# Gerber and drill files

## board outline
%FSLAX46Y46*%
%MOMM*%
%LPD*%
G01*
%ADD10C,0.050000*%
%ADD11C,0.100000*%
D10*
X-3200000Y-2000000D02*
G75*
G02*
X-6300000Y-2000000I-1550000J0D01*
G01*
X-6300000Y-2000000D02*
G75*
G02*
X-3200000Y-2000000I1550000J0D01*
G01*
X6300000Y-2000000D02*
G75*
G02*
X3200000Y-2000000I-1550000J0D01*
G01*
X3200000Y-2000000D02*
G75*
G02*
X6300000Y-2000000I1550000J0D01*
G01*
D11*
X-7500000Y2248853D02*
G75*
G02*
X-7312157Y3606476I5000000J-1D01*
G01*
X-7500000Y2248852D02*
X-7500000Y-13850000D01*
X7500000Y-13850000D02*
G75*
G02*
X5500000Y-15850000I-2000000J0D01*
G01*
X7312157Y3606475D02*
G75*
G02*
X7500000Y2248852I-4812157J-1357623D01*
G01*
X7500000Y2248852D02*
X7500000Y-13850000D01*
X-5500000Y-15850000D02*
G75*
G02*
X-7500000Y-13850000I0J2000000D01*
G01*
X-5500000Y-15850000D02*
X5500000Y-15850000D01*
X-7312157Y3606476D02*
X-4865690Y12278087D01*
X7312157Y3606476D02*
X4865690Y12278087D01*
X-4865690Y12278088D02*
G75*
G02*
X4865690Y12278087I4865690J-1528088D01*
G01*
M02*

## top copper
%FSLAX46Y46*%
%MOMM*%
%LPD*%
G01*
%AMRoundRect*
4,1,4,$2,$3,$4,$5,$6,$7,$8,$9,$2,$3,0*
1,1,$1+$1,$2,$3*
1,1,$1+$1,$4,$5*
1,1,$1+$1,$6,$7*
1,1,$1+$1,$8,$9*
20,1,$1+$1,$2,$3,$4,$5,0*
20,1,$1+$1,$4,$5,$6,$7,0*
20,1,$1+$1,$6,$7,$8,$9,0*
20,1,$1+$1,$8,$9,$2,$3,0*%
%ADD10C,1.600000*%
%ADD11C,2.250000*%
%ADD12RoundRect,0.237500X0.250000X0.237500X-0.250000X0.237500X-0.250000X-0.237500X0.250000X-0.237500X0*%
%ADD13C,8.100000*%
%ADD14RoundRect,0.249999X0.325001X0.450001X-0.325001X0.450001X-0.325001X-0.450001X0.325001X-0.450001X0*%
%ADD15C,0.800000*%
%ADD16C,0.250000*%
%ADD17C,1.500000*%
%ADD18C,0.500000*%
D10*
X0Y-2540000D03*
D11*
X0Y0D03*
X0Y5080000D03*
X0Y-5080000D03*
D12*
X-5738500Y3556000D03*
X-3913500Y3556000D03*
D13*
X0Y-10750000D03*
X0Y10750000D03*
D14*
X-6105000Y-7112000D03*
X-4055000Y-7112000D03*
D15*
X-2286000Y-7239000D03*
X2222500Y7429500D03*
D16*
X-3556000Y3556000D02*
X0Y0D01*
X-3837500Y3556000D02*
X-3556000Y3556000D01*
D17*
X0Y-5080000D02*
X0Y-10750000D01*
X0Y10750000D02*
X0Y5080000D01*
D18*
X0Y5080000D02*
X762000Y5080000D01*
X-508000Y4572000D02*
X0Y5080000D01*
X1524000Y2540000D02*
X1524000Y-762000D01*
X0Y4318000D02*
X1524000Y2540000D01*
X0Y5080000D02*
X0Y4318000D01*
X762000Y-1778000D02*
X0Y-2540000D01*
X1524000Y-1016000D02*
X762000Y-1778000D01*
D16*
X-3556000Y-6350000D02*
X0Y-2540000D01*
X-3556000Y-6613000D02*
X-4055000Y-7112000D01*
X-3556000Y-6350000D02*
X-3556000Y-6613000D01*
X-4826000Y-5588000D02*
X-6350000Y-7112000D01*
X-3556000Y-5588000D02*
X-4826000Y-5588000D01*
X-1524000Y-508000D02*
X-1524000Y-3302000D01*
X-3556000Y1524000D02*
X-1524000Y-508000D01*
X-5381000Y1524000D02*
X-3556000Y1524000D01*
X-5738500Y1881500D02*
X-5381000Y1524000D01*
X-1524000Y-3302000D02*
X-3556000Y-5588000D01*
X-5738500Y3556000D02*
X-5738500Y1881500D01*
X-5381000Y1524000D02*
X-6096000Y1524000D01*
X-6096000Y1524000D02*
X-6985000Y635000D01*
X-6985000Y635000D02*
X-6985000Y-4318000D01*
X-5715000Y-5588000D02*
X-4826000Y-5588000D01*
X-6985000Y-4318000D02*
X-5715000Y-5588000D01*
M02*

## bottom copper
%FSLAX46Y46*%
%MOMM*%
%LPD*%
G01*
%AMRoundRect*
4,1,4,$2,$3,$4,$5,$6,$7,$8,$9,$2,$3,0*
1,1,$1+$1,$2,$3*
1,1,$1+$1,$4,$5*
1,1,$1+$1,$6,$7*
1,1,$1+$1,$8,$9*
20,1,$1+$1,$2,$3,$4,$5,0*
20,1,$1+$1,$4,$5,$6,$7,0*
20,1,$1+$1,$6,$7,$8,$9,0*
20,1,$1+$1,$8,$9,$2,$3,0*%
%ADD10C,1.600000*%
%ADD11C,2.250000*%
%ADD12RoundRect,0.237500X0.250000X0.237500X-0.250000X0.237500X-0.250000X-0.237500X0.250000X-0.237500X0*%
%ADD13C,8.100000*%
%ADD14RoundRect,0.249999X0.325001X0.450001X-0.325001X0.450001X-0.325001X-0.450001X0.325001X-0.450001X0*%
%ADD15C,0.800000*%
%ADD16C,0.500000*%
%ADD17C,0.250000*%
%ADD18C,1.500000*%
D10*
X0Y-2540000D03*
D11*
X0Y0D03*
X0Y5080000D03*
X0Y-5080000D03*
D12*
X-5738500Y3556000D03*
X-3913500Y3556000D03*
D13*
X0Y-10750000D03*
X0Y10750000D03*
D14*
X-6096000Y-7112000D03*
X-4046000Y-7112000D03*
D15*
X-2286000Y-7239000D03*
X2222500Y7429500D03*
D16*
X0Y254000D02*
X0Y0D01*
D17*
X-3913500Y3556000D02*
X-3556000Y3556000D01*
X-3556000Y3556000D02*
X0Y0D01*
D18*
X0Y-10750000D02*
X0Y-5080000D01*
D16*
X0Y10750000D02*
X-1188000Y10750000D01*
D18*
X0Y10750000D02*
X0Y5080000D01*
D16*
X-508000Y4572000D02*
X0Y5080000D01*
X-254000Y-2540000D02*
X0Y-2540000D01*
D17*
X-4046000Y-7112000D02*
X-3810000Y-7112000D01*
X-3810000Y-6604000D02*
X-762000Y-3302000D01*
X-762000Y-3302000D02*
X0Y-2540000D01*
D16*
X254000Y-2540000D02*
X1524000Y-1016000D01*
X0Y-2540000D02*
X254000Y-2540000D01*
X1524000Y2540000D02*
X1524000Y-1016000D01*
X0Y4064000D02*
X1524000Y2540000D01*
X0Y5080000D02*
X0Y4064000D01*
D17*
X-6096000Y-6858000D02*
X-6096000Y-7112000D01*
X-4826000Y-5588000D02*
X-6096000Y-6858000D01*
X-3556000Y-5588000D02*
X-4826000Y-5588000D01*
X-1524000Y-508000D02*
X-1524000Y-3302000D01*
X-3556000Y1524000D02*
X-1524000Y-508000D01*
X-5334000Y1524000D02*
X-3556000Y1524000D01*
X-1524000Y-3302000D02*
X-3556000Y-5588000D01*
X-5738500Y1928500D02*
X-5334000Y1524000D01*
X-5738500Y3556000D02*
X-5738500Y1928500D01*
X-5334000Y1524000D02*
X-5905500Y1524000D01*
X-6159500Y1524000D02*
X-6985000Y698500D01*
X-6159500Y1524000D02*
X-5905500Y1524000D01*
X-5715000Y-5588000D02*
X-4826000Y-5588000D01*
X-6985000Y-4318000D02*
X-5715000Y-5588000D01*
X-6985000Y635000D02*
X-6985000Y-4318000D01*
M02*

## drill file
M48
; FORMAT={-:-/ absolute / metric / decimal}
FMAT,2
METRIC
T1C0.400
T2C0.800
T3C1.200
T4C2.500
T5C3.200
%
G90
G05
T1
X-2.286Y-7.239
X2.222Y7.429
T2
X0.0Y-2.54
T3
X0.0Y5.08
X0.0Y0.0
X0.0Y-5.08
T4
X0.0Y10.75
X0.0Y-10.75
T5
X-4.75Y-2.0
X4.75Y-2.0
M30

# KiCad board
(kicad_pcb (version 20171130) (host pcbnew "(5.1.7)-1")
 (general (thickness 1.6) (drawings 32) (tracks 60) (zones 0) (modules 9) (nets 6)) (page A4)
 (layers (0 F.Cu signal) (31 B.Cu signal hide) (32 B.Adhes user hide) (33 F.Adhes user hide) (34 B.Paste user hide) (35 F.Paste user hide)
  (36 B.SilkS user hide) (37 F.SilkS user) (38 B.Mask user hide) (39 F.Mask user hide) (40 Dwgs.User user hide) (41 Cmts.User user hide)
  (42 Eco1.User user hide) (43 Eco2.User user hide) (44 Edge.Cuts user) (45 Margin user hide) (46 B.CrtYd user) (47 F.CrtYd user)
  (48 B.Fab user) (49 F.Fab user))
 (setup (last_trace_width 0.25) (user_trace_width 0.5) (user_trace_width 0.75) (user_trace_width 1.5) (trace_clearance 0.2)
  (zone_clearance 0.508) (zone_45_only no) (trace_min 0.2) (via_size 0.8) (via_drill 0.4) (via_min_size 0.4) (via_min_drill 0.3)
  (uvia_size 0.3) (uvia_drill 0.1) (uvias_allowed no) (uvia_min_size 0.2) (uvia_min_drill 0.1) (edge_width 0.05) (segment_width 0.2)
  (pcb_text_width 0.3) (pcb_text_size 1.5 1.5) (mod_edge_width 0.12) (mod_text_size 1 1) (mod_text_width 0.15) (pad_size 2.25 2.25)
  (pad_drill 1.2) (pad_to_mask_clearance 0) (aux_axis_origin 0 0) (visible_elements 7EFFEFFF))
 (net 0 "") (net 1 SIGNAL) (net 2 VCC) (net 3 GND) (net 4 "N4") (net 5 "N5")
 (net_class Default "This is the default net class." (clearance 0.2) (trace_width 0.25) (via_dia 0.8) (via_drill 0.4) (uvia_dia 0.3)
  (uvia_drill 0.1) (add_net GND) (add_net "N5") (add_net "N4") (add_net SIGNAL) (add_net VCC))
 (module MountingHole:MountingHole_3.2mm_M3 (layer F.Cu) (at 4.75 2)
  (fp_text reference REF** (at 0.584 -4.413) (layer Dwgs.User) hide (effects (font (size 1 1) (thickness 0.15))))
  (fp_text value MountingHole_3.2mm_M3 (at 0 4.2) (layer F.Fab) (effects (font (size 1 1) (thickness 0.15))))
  (pad 1 np_thru_hole circle (at 0 0) (size 3.2 3.2) (drill 3.2) (layers *.Cu *.Mask)))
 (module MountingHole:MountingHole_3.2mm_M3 (layer F.Cu) (at -4.75 2)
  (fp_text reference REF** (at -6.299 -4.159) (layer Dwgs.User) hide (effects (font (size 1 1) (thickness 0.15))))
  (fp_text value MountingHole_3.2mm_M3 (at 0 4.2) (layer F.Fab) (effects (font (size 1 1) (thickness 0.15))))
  (pad 1 np_thru_hole circle (at 0 0) (size 3.2 3.2) (drill 3.2) (layers *.Cu *.Mask)))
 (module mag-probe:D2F (layer F.Cu) (at 0 0 270)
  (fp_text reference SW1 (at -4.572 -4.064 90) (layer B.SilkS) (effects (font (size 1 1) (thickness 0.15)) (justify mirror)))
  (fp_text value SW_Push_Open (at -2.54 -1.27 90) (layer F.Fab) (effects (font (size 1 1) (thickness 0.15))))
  (pad 4 thru_hole circle (at 2.54 0 270) (size 1.6 1.6) (drill 0.8) (layers *.Cu *.Mask) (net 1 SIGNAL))
  (pad 3 thru_hole circle (at 0 0 270) (size 2.25 2.25) (drill 1.2) (layers *.Cu *.Mask) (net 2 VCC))
  (pad 2 thru_hole circle (at -5.08 0 270) (size 2.25 2.25) (drill 1.2) (layers *.Cu *.Mask) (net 1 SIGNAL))
  (pad 1 thru_hole circle (at 5.08 0 270) (size 2.25 2.25) (drill 1.2) (layers *.Cu *.Mask) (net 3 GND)))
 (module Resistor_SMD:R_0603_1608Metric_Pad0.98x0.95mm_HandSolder (layer B.Cu) (at -4.826 -3.556 180)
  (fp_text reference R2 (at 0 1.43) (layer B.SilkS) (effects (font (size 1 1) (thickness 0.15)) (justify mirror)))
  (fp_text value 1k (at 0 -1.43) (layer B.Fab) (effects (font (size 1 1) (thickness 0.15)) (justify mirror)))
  (pad 2 smd roundrect (at 0.9125 0 180) (size 0.975 0.95) (layers B.Cu B.Paste B.Mask) (roundrect_rratio 0.25) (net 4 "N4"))
  (pad 1 smd roundrect (at -0.9125 0 180) (size 0.975 0.95) (layers B.Cu B.Paste B.Mask) (roundrect_rratio 0.25) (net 2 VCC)))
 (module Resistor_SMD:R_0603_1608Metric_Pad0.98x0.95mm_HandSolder (layer F.Cu) (at -4.826 -3.556 180)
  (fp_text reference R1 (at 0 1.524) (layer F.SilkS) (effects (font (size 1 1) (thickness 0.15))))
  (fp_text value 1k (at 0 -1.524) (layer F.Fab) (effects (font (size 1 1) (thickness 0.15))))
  (pad 2 smd roundrect (at 0.9125 0 180) (size 0.975 0.95) (layers F.Cu F.Paste F.Mask) (roundrect_rratio 0.25) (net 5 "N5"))
  (pad 1 smd roundrect (at -0.9125 0 180) (size 0.975 0.95) (layers F.Cu F.Paste F.Mask) (roundrect_rratio 0.25) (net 2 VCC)))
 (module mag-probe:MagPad (layer F.Cu) (at 0 10.75)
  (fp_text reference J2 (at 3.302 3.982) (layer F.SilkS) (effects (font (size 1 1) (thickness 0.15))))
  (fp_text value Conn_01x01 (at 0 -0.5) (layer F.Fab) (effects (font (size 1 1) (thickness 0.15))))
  (pad 1 thru_hole circle (at 0 0) (size 8.1 8.1) (drill 2.5) (layers *.Cu *.Mask) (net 3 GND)))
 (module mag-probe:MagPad (layer F.Cu) (at 0 -10.75)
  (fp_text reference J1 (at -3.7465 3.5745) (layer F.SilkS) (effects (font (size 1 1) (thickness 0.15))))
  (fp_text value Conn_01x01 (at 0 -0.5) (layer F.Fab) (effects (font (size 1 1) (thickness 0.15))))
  (pad 1 thru_hole circle (at 0 0) (size 8.1 8.1) (drill 2.5) (layers *.Cu *.Mask) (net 1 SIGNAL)))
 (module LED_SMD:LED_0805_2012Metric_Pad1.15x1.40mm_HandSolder (layer B.Cu) (at -5.071 7.112 180)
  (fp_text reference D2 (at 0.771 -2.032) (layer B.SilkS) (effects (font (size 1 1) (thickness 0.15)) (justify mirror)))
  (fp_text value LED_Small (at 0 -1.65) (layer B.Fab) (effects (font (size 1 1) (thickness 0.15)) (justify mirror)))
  (pad 2 smd roundrect (at 1.025 0 180) (size 1.15 1.4) (layers B.Cu B.Paste B.Mask) (roundrect_rratio 0.2173904347826087) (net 4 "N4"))
  (pad 1 smd roundrect (at -1.025 0 180) (size 1.15 1.4) (layers B.Cu B.Paste B.Mask) (roundrect_rratio 0.2173904347826087) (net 1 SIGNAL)))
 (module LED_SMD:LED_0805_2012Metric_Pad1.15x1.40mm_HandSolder (layer F.Cu) (at -5.08 7.112 180)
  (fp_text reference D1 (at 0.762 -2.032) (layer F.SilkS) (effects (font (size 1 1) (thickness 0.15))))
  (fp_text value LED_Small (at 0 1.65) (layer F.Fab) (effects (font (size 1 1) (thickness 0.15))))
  (pad 2 smd roundrect (at 1.025 0 180) (size 1.15 1.4) (layers F.Cu F.Paste F.Mask) (roundrect_rratio 0.2173904347826087) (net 5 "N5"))
  (pad 1 smd roundrect (at -1.025 0 180) (size 1.15 1.4) (layers F.Cu F.Paste F.Mask) (roundrect_rratio 0.2173904347826087) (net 1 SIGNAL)))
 (gr_circle (center -4.75 2) (end -3.2 2) (layer Edge.Cuts) (width 0.05))
 (gr_circle (center 4.75 2) (end 6.3 2) (layer Edge.Cuts) (width 0.05))
 (gr_arc (start -2.5 -2.248852) (end -7.312157 -3.606476) (angle -15.75501346) (layer Edge.Cuts) (width 0.1))
 (gr_line (start -7.5 -2.248852) (end -7.5 13.85) (layer Edge.Cuts) (width 0.1))
 (gr_arc (start 5.5 13.85) (end 5.5 15.85) (angle -90) (layer Edge.Cuts) (width 0.1))
 (gr_arc (start 2.5 -2.248852) (end 7.5 -2.248852) (angle -15.75501346) (layer Edge.Cuts) (width 0.1))
 (gr_line (start 7.5 -2.248852) (end 7.5 13.85) (layer Edge.Cuts) (width 0.1))
 (gr_arc (start -5.5 13.85) (end -7.5 13.85) (angle -90) (layer Edge.Cuts) (width 0.1))
 (gr_line (start -5.5 15.85) (end 5.5 15.85) (layer Edge.Cuts) (width 0.1))
 (gr_line (start -7.312157 -3.606476) (end -4.86569 -12.278087) (layer Edge.Cuts) (width 0.1))
 (gr_line (start 7.312157 -3.606476) (end 4.86569 -12.278087) (layer Edge.Cuts) (width 0.1))
 (gr_arc (start 0 -10.75) (end 4.86569 -12.278087) (angle -145.1298326) (layer Edge.Cuts) (width 0.1))
 (via (at -2.286 7.239) (size 0.8) (drill 0.4) (layers F.Cu B.Cu) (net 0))
 (segment (start 0 -0.254) (end 0 0) (width 0.5) (layer B.Cu) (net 2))
 (segment (start -3.9135 -3.556) (end -3.556 -3.556) (width 0.25) (layer B.Cu) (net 2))
 (segment (start -3.556 -3.556) (end 0 0) (width 0.25) (layer B.Cu) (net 2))
 (segment (start -3.556 -3.556) (end 0 0) (width 0.25) (layer F.Cu) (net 2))
 (segment (start -3.8375 -3.556) (end -3.556 -3.556) (width 0.25) (layer F.Cu) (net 2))
 (segment (start 0 10.75) (end 0 5.08) (width 1.5) (layer B.Cu) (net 3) (status 30))
 (segment (start 0 5.08) (end 0 10.75) (width 1.5) (layer F.Cu) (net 3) (status 30))
 (via (at 2.2225 -7.4295) (size 0.8) (drill 0.4) (layers F.Cu B.Cu) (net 1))
 (segment (start 0 -10.75) (end -1.188 -10.75) (width 0.5) (layer B.Cu) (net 1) (status 30))
 (segment (start 0 -10.75) (end 0 -5.08) (width 1.5) (layer B.Cu) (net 1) (status 30))
 (segment (start -0.508 -4.572) (end 0 -5.08) (width 0.5) (layer B.Cu) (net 1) (status 30))
 (segment (start 0 -10.75) (end 0 -5.08) (width 1.5) (layer F.Cu) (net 1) (status 30))
 (segment (start 0 -5.08) (end 0.762 -5.08) (width 0.5) (layer F.Cu) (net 1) (status 30))
 (segment (start -0.508 -4.572) (end 0 -5.08) (width 0.5) (layer F.Cu) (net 1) (status 30))
 (segment (start 1.524 -2.54) (end 1.524 0.762) (width 0.5) (layer F.Cu) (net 1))
 (segment (start -0.254 2.54) (end 0 2.54) (width 0.5) (layer B.Cu) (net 1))
 (segment (start -4.046 7.112) (end -3.81 7.112) (width 0.25) (layer B.Cu) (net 1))
 (segment (start -3.81 6.604) (end -0.762 3.302) (width 0.25) (layer B.Cu) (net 1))
 (segment (start -0.762 3.302) (end 0 2.54) (width 0.25) (layer B.Cu) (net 1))
 (segment (start 0.254 2.54) (end 1.524 1.016) (width 0.5) (layer B.Cu) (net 1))
 (segment (start 0 2.54) (end 0.254 2.54) (width 0.5) (layer B.Cu) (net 1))
 (segment (start 1.524 -2.54) (end 1.524 1.016) (width 0.5) (layer B.Cu) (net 1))
 (segment (start 0 -4.064) (end 1.524 -2.54) (width 0.5) (layer B.Cu) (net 1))
 (segment (start 0 -5.08) (end 0 -4.064) (width 0.5) (layer B.Cu) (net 1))
 (segment (start 0 -4.318) (end 1.524 -2.54) (width 0.5) (layer F.Cu) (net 1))
 (segment (start 0 -5.08) (end 0 -4.318) (width 0.5) (layer F.Cu) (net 1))
 (segment (start 0.762 1.778) (end 0 2.54) (width 0.5) (layer F.Cu) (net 1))
 (segment (start 1.524 1.016) (end 0.762 1.778) (width 0.5) (layer F.Cu) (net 1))
 (segment (start -3.556 6.35) (end 0 2.54) (width 0.25) (layer F.Cu) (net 1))
 (segment (start -3.556 6.613) (end -4.055 7.112) (width 0.25) (layer F.Cu) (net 1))
 (segment (start -3.556 6.35) (end -3.556 6.613) (width 0.25) (layer F.Cu) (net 1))
 (segment (start -4.826 5.588) (end -6.35 7.112) (width 0.25) (layer F.Cu) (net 5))
 (segment (start -3.556 5.588) (end -4.826 5.588) (width 0.25) (layer F.Cu) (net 5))
 (segment (start -1.524 0.508) (end -1.524 3.302) (width 0.25) (layer F.Cu) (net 5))
 (segment (start -3.556 -1.524) (end -1.524 0.508) (width 0.25) (layer F.Cu) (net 5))
 (segment (start -5.381 -1.524) (end -3.556 -1.524) (width 0.25) (layer F.Cu) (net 5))
 (segment (start -5.7385 -1.8815) (end -5.381 -1.524) (width 0.25) (layer F.Cu) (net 5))
 (segment (start -1.524 3.302) (end -3.556 5.588) (width 0.25) (layer F.Cu) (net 5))
 (segment (start -5.7385 -3.556) (end -5.7385 -1.8815) (width 0.25) (layer F.Cu) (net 5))
 (segment (start -5.381 -1.524) (end -6.096 -1.524) (width 0.25) (layer F.Cu) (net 5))
 (segment (start -6.096 -1.524) (end -6.985 -0.635) (width 0.25) (layer F.Cu) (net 5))
 (segment (start -6.985 -0.635) (end -6.985 4.318) (width 0.25) (layer F.Cu) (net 5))
 (segment (start -5.715 5.588) (end -4.826 5.588) (width 0.25) (layer F.Cu) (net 5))
 (segment (start -6.985 4.318) (end -5.715 5.588) (width 0.25) (layer F.Cu) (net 5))
 (segment (start -6.096 6.858) (end -6.096 7.112) (width 0.25) (layer B.Cu) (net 4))
 (segment (start -4.826 5.588) (end -6.096 6.858) (width 0.25) (layer B.Cu) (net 4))
 (segment (start -3.556 5.588) (end -4.826 5.588) (width 0.25) (layer B.Cu) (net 4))
 (segment (start -1.524 0.508) (end -1.524 3.302) (width 0.25) (layer B.Cu) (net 4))
 (segment (start -3.556 -1.524) (end -1.524 0.508) (width 0.25) (layer B.Cu) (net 4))
 (segment (start -5.334 -1.524) (end -3.556 -1.524) (width 0.25) (layer B.Cu) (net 4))
 (segment (start -1.524 3.302) (end -3.556 5.588) (width 0.25) (layer B.Cu) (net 4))
 (segment (start -5.7385 -1.9285) (end -5.334 -1.524) (width 0.25) (layer B.Cu) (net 4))
 (segment (start -5.7385 -3.556) (end -5.7385 -1.9285) (width 0.25) (layer B.Cu) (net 4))
 (segment (start -5.334 -1.524) (end -5.9055 -1.524) (width 0.25) (layer B.Cu) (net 4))
 (segment (start -6.1595 -1.524) (end -6.985 -0.6985) (width 0.25) (layer B.Cu) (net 4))
 (segment (start -6.1595 -1.524) (end -5.9055 -1.524) (width 0.25) (layer B.Cu) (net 4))
 (segment (start -5.715 5.588) (end -4.826 5.588) (width 0.25) (layer B.Cu) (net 4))
 (segment (start -6.985 4.318) (end -5.715 5.588) (width 0.25) (layer B.Cu) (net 4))
 (segment (start -6.985 -0.635) (end -6.985 4.318) (width 0.25) (layer B.Cu) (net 4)))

